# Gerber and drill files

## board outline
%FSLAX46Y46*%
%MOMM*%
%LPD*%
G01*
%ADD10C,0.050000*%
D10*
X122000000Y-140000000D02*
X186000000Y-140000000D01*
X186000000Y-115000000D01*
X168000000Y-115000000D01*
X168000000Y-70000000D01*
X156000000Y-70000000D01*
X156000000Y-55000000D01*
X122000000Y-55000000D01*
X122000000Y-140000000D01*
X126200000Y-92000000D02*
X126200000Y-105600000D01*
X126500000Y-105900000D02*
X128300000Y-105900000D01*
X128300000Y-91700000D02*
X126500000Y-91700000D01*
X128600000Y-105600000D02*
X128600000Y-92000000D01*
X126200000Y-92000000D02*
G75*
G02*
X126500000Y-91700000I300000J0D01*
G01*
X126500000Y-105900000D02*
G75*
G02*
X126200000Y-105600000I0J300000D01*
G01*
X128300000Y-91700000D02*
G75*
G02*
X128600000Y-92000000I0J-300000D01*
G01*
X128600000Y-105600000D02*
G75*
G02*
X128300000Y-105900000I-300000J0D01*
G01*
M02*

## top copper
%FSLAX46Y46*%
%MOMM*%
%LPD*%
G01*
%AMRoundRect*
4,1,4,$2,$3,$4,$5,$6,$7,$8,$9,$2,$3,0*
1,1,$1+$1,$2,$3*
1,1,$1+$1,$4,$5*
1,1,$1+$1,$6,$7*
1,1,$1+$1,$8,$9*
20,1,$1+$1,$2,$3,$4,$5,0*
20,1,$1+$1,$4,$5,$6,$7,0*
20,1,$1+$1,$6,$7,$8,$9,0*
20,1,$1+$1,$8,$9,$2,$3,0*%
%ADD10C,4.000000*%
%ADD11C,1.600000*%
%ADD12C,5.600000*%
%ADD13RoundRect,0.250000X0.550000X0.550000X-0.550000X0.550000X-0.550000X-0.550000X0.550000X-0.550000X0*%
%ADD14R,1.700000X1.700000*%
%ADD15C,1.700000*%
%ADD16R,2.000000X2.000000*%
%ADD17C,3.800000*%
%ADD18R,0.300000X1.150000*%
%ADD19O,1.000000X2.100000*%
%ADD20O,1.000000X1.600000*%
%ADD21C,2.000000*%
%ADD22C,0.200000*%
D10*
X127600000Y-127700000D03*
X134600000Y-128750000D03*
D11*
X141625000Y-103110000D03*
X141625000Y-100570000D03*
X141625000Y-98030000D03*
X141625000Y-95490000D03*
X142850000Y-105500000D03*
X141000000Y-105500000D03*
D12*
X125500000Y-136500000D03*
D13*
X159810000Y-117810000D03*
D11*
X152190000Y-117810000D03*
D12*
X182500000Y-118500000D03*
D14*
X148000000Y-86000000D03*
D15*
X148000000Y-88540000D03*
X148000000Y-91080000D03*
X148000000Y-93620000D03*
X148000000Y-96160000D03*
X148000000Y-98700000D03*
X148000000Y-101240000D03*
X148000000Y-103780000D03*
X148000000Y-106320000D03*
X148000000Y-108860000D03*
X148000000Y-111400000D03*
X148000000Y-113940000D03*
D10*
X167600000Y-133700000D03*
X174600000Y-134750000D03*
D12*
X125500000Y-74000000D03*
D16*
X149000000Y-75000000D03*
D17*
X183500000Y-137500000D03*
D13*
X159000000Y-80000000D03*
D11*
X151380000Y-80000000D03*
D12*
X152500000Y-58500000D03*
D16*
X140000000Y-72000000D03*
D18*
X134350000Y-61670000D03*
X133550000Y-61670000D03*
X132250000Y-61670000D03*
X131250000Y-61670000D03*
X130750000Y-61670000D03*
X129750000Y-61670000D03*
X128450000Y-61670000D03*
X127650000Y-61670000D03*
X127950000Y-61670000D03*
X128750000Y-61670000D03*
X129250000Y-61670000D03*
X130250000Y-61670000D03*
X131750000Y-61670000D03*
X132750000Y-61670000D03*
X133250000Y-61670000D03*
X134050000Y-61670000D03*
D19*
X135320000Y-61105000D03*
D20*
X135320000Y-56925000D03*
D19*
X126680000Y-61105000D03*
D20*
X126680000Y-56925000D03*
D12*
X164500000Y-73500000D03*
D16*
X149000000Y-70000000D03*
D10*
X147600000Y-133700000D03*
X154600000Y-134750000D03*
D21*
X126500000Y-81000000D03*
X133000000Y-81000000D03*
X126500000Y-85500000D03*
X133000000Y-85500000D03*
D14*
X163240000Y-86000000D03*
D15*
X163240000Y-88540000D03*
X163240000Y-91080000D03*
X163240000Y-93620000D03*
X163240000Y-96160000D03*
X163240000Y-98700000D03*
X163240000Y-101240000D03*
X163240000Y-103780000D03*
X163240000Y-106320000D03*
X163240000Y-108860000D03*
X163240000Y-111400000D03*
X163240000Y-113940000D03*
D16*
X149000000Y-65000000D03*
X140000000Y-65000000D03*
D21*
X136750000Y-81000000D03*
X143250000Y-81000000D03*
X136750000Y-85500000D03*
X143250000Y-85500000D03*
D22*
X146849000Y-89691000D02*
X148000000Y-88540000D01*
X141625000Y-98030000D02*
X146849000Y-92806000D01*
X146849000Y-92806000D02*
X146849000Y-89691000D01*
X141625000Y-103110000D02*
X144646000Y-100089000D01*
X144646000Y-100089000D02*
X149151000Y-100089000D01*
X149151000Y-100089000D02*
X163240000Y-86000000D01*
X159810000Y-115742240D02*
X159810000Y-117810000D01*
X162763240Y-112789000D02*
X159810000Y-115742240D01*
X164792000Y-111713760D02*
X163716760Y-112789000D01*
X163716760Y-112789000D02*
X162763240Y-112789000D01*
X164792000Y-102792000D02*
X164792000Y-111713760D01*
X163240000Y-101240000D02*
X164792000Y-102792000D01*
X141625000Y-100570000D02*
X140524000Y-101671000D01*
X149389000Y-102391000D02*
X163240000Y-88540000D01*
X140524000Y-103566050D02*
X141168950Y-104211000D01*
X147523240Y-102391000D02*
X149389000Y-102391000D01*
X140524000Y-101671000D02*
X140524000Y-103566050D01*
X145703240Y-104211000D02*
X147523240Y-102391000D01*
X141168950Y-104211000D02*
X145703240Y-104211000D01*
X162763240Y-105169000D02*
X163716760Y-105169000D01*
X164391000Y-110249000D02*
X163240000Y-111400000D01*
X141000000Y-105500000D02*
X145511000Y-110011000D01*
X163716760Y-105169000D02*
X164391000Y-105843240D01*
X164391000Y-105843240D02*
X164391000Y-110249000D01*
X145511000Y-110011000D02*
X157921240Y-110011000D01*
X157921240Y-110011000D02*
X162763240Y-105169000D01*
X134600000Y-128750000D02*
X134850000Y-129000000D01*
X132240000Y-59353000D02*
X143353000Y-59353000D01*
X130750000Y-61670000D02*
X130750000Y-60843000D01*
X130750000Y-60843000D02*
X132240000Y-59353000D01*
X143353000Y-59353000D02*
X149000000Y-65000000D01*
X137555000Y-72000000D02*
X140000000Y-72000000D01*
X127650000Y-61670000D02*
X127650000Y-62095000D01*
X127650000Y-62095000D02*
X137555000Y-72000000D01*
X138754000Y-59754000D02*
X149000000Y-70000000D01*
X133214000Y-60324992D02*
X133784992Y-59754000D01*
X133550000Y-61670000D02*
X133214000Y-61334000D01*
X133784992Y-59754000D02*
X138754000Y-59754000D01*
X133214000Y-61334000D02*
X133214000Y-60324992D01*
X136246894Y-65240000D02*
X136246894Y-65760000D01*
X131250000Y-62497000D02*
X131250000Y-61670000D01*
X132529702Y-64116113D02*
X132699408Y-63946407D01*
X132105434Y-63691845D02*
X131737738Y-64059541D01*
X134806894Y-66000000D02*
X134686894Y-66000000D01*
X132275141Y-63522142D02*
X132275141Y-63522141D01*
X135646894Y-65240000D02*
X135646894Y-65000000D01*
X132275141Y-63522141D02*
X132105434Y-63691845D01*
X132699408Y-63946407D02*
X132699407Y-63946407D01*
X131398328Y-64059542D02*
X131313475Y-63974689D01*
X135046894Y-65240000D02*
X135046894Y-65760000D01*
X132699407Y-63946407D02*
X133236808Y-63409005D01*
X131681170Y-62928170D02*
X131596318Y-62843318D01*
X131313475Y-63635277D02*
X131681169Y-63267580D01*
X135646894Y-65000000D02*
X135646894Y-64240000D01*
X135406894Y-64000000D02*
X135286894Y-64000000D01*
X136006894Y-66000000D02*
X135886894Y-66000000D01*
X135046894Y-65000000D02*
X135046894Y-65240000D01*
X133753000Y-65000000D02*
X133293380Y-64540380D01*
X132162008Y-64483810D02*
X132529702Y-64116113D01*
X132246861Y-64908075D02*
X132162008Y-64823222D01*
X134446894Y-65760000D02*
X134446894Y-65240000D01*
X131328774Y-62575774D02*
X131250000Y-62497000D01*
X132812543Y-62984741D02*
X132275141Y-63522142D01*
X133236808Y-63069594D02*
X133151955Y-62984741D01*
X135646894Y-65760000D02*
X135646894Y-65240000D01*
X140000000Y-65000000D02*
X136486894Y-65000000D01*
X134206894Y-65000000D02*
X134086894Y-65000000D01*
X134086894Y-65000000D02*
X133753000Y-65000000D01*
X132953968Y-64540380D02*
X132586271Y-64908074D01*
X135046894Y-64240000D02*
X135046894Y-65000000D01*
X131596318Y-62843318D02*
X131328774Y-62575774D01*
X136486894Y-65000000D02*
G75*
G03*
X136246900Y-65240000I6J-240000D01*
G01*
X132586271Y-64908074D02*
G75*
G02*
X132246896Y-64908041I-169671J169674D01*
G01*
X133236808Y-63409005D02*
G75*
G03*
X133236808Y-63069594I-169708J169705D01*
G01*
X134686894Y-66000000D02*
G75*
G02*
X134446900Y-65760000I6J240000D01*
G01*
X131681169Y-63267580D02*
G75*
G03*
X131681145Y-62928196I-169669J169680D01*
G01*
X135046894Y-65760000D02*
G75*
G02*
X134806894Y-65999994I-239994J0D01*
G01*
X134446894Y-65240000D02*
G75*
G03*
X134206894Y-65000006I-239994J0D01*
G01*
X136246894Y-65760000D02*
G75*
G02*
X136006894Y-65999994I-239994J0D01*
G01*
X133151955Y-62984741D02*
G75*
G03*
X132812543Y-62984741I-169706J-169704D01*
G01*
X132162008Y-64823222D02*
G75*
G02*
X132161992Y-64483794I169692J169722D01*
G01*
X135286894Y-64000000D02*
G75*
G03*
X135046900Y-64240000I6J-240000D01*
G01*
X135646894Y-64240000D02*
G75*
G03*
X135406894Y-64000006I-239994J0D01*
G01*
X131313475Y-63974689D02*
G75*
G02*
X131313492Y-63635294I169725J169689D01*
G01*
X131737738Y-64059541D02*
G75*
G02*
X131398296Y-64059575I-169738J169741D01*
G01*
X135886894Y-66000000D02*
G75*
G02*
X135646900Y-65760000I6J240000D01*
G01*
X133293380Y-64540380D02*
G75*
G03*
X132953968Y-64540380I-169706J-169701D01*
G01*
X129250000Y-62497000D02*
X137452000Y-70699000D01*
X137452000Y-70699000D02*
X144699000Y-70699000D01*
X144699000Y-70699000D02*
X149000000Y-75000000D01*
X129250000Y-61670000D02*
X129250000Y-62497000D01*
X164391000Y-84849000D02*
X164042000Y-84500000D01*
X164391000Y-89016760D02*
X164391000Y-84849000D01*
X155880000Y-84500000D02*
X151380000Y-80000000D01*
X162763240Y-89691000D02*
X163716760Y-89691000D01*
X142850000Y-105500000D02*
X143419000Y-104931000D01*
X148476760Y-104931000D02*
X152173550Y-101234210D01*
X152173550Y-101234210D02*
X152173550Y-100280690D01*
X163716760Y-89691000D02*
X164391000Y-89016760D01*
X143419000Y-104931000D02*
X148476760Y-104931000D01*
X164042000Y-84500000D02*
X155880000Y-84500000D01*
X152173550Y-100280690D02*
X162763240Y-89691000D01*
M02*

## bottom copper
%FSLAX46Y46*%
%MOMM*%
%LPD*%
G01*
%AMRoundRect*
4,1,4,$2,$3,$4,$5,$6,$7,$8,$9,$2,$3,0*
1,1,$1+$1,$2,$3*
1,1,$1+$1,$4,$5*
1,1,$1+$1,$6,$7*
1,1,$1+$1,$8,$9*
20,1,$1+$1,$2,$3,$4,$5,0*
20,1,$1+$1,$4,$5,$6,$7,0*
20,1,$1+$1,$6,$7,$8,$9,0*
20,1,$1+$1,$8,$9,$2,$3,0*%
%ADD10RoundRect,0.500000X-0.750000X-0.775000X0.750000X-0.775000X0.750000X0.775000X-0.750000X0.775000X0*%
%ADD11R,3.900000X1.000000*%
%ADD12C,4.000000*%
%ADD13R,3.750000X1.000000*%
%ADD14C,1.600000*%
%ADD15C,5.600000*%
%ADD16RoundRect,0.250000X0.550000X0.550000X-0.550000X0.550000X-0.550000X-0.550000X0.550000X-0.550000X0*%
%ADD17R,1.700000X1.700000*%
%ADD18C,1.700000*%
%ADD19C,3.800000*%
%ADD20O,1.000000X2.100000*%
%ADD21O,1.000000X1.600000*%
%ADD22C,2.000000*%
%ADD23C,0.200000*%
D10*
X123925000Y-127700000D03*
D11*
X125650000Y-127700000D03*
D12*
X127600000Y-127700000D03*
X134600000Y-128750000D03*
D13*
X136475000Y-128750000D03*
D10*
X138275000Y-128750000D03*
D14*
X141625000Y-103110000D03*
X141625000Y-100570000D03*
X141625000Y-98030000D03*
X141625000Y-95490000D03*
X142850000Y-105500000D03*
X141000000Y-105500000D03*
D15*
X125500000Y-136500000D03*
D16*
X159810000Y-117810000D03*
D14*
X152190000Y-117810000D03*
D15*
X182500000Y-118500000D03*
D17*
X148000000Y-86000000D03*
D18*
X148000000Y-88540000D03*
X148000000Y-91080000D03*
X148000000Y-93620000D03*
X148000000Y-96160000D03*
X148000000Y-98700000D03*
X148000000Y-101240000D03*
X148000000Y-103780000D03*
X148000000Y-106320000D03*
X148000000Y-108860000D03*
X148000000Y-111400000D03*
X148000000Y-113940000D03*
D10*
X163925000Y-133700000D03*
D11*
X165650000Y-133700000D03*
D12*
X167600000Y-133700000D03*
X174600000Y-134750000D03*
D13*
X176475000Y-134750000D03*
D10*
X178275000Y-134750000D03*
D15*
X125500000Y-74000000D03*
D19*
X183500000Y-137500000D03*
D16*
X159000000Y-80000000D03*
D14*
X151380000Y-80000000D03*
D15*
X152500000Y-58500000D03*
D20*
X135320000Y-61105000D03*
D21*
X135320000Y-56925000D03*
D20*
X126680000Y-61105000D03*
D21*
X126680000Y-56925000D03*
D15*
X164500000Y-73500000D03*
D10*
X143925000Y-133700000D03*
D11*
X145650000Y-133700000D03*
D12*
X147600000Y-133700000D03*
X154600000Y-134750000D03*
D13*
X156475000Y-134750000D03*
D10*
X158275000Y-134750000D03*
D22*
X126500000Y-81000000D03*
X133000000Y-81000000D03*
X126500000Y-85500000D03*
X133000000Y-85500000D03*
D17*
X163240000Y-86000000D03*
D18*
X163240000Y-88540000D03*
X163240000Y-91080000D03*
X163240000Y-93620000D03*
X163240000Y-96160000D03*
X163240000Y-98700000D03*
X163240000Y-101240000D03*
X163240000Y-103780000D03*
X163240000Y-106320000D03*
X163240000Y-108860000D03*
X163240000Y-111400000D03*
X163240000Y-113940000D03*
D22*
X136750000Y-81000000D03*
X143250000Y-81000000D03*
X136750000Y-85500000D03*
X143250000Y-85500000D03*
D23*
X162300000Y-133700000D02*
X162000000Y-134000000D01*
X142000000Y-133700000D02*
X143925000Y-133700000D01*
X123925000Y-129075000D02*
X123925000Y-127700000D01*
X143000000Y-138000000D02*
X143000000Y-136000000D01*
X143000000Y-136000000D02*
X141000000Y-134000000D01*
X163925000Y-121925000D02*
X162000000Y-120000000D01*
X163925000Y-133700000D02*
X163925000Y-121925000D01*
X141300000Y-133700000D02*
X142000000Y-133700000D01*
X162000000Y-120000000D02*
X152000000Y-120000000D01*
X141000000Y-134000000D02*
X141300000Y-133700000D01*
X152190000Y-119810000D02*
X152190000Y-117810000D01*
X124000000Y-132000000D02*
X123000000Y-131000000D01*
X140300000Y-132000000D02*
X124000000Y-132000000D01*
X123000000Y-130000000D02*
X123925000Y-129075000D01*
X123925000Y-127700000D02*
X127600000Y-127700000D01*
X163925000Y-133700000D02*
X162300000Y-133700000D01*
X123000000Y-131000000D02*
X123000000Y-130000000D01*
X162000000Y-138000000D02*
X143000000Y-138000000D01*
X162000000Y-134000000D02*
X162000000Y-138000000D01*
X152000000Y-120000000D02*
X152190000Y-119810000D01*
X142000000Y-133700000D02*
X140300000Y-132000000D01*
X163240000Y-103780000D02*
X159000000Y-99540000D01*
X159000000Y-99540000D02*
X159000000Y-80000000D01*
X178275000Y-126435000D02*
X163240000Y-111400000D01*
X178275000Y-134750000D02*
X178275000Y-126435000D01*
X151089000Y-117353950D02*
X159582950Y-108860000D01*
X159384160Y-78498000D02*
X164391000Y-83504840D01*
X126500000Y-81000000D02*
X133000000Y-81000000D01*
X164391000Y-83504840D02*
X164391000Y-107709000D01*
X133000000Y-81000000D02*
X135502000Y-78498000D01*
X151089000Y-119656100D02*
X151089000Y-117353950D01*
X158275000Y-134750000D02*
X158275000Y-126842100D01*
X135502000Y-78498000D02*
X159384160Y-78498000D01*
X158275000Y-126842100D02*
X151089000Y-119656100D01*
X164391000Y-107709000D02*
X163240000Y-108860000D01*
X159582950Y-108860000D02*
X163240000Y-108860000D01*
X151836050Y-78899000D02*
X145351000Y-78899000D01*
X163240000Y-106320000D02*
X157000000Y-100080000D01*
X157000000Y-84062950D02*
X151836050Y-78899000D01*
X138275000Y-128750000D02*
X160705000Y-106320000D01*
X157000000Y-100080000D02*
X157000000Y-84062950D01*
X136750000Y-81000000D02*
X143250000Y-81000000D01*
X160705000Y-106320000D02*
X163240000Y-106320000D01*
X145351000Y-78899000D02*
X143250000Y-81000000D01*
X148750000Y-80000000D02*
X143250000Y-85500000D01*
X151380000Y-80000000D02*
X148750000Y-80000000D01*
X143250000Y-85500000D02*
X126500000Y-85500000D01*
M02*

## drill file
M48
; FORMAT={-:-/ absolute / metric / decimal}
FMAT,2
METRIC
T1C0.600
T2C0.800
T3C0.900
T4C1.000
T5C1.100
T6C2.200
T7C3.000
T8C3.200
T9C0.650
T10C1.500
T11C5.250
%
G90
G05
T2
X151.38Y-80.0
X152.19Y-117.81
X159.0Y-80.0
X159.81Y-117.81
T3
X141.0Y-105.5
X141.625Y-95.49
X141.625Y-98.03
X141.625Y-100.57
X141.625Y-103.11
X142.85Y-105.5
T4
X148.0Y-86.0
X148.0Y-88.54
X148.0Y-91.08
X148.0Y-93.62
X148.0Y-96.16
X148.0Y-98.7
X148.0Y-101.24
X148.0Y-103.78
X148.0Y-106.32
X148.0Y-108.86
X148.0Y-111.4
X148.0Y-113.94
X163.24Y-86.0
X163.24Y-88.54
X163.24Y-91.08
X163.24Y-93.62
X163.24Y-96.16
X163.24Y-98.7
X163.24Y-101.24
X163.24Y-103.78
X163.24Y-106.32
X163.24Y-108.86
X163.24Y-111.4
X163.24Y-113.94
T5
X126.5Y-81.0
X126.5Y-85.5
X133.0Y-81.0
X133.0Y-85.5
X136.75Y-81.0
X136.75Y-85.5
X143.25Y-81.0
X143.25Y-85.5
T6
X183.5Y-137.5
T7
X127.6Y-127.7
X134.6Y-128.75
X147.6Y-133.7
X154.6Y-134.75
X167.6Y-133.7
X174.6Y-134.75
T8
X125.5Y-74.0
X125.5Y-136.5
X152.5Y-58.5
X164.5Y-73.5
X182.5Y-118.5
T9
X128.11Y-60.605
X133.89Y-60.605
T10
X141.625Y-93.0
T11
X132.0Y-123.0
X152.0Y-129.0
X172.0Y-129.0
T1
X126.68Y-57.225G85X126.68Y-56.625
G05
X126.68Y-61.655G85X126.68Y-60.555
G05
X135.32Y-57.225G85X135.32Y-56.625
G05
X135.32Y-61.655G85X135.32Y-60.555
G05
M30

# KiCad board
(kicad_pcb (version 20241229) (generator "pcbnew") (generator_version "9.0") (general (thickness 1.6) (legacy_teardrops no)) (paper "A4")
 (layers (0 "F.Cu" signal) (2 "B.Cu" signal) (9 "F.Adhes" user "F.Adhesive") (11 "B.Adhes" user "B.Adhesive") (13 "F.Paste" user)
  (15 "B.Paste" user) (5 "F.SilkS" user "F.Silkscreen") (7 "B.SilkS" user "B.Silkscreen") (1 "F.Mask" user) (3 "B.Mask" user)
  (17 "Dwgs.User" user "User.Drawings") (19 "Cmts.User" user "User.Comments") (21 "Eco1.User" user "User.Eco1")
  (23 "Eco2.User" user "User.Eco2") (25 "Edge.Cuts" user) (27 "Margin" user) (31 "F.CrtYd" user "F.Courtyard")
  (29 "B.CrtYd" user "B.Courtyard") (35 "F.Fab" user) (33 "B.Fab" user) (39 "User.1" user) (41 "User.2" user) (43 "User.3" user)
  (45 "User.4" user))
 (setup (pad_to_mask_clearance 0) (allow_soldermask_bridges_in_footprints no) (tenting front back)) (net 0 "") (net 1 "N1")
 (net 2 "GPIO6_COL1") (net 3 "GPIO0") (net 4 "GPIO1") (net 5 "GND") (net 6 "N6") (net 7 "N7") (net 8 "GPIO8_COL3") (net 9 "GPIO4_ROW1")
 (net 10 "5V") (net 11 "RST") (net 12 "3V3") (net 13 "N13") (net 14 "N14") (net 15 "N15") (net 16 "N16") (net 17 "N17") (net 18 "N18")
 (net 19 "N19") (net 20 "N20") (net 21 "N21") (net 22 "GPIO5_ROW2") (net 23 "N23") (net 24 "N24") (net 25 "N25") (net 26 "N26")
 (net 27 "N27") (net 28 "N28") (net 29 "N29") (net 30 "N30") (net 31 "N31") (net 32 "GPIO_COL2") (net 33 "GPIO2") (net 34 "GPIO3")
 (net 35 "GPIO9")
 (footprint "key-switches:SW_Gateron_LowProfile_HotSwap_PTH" (layer "F.Cu") (at 132 123)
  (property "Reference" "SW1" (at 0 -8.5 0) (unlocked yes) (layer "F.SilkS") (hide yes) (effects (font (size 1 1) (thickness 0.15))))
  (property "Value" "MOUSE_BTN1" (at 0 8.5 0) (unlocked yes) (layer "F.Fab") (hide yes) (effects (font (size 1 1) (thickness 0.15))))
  (pad "" np_thru_hole circle (at 0 0) (size 5.25 5.25) (drill 5.25) (layers "*.Mask"))
  (pad "1" smd roundrect (at -8.075 4.7) (size 2.5 2.55) (layers "B.Cu" "B.Mask" "B.Paste") (roundrect_rratio 0.2) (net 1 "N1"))
  (pad "1" smd rect (at -6.35 4.7) (size 3.9 1) (layers "B.Cu") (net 1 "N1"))
  (pad "1" thru_hole circle (at -4.4 4.7) (size 4 4) (drill 3) (layers "*.Cu" "B.Mask") (remove_unused_layers no) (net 1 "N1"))
  (pad "2" thru_hole circle (at 2.6 5.75) (size 4 4) (drill 3) (layers "*.Cu" "B.Mask") (remove_unused_layers no) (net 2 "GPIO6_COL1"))
  (pad "2" smd rect (at 4.475 5.75) (size 3.75 1) (layers "B.Cu") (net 2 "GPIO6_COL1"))
  (pad "2" smd roundrect (at 6.275 5.75) (size 2.5 2.55) (layers "B.Cu" "B.Mask" "B.Paste") (roundrect_rratio 0.2) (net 2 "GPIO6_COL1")))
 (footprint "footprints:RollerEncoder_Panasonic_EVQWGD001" (layer "F.Cu") (at 136 99.3 180)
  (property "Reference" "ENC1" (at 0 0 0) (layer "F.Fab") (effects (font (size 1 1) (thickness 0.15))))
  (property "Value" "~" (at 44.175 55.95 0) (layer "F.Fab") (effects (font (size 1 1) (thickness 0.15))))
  (fp_line (start 9.8 7.3) (end 9.8 -6.3) (stroke (width 0.05) (type solid)) (layer "Edge.Cuts"))
  (fp_line (start 9.5 -6.6) (end 7.7 -6.6) (stroke (width 0.05) (type solid)) (layer "Edge.Cuts"))
  (fp_line (start 7.7 7.6) (end 9.5 7.6) (stroke (width 0.05) (type solid)) (layer "Edge.Cuts"))
  (fp_line (start 7.4 -6.3) (end 7.4 7.3) (stroke (width 0.05) (type solid)) (layer "Edge.Cuts"))
  (fp_arc (start 9.8 7.3) (mid 9.712132 7.512132) (end 9.5 7.6) (stroke (width 0.05) (type solid)) (layer "Edge.Cuts"))
  (fp_arc (start 9.5 -6.6) (mid 9.712132 -6.512132) (end 9.8 -6.3) (stroke (width 0.05) (type solid)) (layer "Edge.Cuts"))
  (fp_arc (start 7.7 7.6) (mid 7.487868 7.512132) (end 7.4 7.3) (stroke (width 0.05) (type solid)) (layer "Edge.Cuts"))
  (fp_arc (start 7.4 -6.3) (mid 7.487868 -6.512132) (end 7.7 -6.6) (stroke (width 0.05) (type solid)) (layer "Edge.Cuts"))
  (pad "" np_thru_hole circle (at -5.625 6.3 180) (size 1.5 1.5) (drill 1.5) (layers "*.Cu" "*.Mask"))
  (pad "A" thru_hole circle (at -5.625 -3.81 180) (size 1.6 1.6) (drill 0.9) (layers "*.Cu" "*.Mask") (remove_unused_layers no)
   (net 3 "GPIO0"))
  (pad "B" thru_hole circle (at -5.625 -1.27 180) (size 1.6 1.6) (drill 0.9) (layers "*.Cu" "*.Mask") (remove_unused_layers no)
   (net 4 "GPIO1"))
  (pad "C" thru_hole circle (at -5.625 1.27 180) (size 1.6 1.6) (drill 0.9) (layers "*.Cu" "*.Mask") (remove_unused_layers no) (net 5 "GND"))
  (pad "D" thru_hole circle (at -5.625 3.81 180) (size 1.6 1.6) (drill 0.9) (layers "*.Cu" "*.Mask") (remove_unused_layers no) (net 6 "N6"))
  (pad "S1" thru_hole circle (at -6.85 -6.2 180) (size 1.6 1.6) (drill 0.9) (layers "*.Cu" "*.Mask") (remove_unused_layers no) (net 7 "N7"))
  (pad "S2" thru_hole circle (at -5 -6.2 180) (size 1.6 1.6) (drill 0.9) (layers "*.Cu" "*.Mask") (remove_unused_layers no)
   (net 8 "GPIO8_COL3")))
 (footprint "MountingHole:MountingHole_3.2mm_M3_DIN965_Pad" (layer "F.Cu") (at 125.5 136.5)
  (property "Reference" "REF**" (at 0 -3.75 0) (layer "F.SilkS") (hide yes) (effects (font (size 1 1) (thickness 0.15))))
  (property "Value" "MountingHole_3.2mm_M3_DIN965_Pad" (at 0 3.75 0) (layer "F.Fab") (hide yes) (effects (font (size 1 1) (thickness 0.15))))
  (pad "1" thru_hole circle (at 0 0) (size 5.6 5.6) (drill 3.2) (layers "*.Cu" "*.Mask") (remove_unused_layers no) (zone_connect 2)))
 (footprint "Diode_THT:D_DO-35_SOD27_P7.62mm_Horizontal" (layer "F.Cu") (at 159.81 117.81 180)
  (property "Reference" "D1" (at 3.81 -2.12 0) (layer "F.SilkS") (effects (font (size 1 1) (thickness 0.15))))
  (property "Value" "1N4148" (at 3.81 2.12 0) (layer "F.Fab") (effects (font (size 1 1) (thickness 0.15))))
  (pad "1" thru_hole roundrect (at 0 0 180) (size 1.6 1.6) (drill 0.8) (layers "*.Cu" "*.Mask") (remove_unused_layers no)
   (roundrect_rratio 0.15625) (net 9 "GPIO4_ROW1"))
  (pad "2" thru_hole circle (at 7.62 0 180) (size 1.6 1.6) (drill 0.8) (layers "*.Cu" "*.Mask") (remove_unused_layers no) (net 1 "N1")))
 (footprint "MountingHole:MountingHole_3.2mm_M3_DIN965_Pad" (layer "F.Cu") (at 182.5 118.5)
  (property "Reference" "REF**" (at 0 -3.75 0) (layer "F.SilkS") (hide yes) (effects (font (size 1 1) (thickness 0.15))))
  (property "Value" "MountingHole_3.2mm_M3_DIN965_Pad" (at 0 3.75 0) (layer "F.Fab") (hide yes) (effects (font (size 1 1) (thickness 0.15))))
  (pad "1" thru_hole circle (at 0 0) (size 5.6 5.6) (drill 3.2) (layers "*.Cu" "*.Mask") (remove_unused_layers no) (zone_connect 2)))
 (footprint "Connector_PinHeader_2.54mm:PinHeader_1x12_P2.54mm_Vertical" (layer "F.Cu") (at 148 86)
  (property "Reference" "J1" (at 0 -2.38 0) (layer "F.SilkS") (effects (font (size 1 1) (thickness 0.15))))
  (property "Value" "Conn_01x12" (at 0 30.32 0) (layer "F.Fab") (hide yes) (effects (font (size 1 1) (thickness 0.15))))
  (pad "1" thru_hole rect (at 0 0) (size 1.7 1.7) (drill 1) (layers "*.Cu" "*.Mask") (remove_unused_layers no) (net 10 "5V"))
  (pad "2" thru_hole circle (at 0 2.54) (size 1.7 1.7) (drill 1) (layers "*.Cu" "*.Mask") (remove_unused_layers no) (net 5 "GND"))
  (pad "3" thru_hole circle (at 0 5.08) (size 1.7 1.7) (drill 1) (layers "*.Cu" "*.Mask") (remove_unused_layers no) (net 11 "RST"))
  (pad "4" thru_hole circle (at 0 7.62) (size 1.7 1.7) (drill 1) (layers "*.Cu" "*.Mask") (remove_unused_layers no) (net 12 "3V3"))
  (pad "5" thru_hole circle (at 0 10.16) (size 1.7 1.7) (drill 1) (layers "*.Cu" "*.Mask") (remove_unused_layers no) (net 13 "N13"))
  (pad "6" thru_hole circle (at 0 12.7) (size 1.7 1.7) (drill 1) (layers "*.Cu" "*.Mask") (remove_unused_layers no) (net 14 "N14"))
  (pad "7" thru_hole circle (at 0 15.24) (size 1.7 1.7) (drill 1) (layers "*.Cu" "*.Mask") (remove_unused_layers no) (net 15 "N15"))
  (pad "8" thru_hole circle (at 0 17.78) (size 1.7 1.7) (drill 1) (layers "*.Cu" "*.Mask") (remove_unused_layers no) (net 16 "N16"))
  (pad "9" thru_hole circle (at 0 20.32) (size 1.7 1.7) (drill 1) (layers "*.Cu" "*.Mask") (remove_unused_layers no) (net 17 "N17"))
  (pad "10" thru_hole circle (at 0 22.86) (size 1.7 1.7) (drill 1) (layers "*.Cu" "*.Mask") (remove_unused_layers no) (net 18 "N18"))
  (pad "11" thru_hole circle (at 0 25.4) (size 1.7 1.7) (drill 1) (layers "*.Cu" "*.Mask") (remove_unused_layers no) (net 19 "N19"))
  (pad "12" thru_hole circle (at 0 27.94) (size 1.7 1.7) (drill 1) (layers "*.Cu" "*.Mask") (remove_unused_layers no) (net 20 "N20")))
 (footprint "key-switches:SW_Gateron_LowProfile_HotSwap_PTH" (layer "F.Cu") (at 172 129)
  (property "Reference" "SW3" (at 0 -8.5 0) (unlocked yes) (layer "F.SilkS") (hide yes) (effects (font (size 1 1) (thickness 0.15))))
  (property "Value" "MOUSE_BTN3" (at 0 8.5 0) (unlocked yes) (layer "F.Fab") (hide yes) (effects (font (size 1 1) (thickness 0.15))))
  (pad "" np_thru_hole circle (at 0 0) (size 5.25 5.25) (drill 5.25) (layers "*.Mask"))
  (pad "1" smd roundrect (at -8.075 4.7) (size 2.5 2.55) (layers "B.Cu" "B.Mask" "B.Paste") (roundrect_rratio 0.2) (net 1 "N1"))
  (pad "1" smd rect (at -6.35 4.7) (size 3.9 1) (layers "B.Cu") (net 1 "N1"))
  (pad "1" thru_hole circle (at -4.4 4.7) (size 4 4) (drill 3) (layers "*.Cu" "B.Mask") (remove_unused_layers no) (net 1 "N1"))
  (pad "2" thru_hole circle (at 2.6 5.75) (size 4 4) (drill 3) (layers "*.Cu" "B.Mask") (remove_unused_layers no) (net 8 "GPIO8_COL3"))
  (pad "2" smd rect (at 4.475 5.75) (size 3.75 1) (layers "B.Cu") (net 8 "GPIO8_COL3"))
  (pad "2" smd roundrect (at 6.275 5.75) (size 2.5 2.55) (layers "B.Cu" "B.Mask" "B.Paste") (roundrect_rratio 0.2) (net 8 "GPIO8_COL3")))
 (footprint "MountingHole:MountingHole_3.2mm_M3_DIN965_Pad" (layer "F.Cu") (at 125.5 74)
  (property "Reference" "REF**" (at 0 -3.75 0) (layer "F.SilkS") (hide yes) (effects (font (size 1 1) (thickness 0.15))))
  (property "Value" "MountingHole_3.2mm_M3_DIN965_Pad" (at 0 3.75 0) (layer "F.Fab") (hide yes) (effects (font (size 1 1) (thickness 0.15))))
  (pad "1" thru_hole circle (at 0 0) (size 5.6 5.6) (drill 3.2) (layers "*.Cu" "*.Mask") (remove_unused_layers no) (zone_connect 2)))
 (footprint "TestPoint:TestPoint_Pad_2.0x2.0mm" (layer "F.Cu") (at 149 75)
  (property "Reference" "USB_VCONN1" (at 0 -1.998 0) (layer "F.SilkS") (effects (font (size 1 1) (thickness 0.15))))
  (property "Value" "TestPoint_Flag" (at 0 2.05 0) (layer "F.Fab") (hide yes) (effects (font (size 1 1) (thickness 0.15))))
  (pad "1" smd rect (at 0 0) (size 2 2) (layers "F.Cu" "F.Mask") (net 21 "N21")))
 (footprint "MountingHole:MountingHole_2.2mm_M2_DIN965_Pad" (layer "F.Cu") (at 183.5 137.5)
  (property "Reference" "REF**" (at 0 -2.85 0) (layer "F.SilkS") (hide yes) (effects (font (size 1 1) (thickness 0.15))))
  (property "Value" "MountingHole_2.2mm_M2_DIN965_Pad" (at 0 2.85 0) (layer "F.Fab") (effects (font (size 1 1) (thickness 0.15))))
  (pad "1" thru_hole circle (at 0 0) (size 3.8 3.8) (drill 2.2) (layers "*.Cu" "*.Mask") (remove_unused_layers no) (zone_connect 2)))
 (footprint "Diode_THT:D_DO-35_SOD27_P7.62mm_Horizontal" (layer "F.Cu") (at 159 80 180)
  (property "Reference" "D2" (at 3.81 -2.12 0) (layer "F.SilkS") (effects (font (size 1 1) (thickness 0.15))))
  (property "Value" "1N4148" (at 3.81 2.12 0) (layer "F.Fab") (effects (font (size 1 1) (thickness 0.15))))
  (pad "1" thru_hole roundrect (at 0 0 180) (size 1.6 1.6) (drill 0.8) (layers "*.Cu" "*.Mask") (remove_unused_layers no)
   (roundrect_rratio 0.15625) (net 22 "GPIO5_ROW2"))
  (pad "2" thru_hole circle (at 7.62 0 180) (size 1.6 1.6) (drill 0.8) (layers "*.Cu" "*.Mask") (remove_unused_layers no) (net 7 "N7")))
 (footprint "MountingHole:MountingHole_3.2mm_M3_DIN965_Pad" (layer "F.Cu") (at 152.5 58.5)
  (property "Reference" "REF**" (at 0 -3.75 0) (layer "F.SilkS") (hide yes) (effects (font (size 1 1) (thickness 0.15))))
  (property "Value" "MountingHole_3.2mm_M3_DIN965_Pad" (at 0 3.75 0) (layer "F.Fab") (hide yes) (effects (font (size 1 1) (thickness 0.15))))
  (pad "1" thru_hole circle (at 0 0) (size 5.6 5.6) (drill 3.2) (layers "*.Cu" "*.Mask") (remove_unused_layers no) (zone_connect 2)))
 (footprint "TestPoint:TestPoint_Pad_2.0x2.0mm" (layer "F.Cu") (at 140 72)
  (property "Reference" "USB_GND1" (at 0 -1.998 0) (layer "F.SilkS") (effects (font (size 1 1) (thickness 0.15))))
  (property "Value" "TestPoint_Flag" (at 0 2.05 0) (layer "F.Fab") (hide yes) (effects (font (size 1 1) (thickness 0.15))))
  (pad "1" smd rect (at 0 0) (size 2 2) (layers "F.Cu" "F.Mask") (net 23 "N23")))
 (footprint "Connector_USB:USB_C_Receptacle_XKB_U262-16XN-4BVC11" (layer "F.Cu") (at 131 58 180)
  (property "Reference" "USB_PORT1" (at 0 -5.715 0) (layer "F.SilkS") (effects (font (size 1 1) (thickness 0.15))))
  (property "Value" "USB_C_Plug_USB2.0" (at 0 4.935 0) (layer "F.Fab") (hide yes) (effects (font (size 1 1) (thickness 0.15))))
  (pad "" np_thru_hole circle (at -2.89 -2.605 180) (size 0.65 0.65) (drill 0.65) (layers "*.Cu" "*.Mask"))
  (pad "" np_thru_hole circle (at 2.89 -2.605 180) (size 0.65 0.65) (drill 0.65) (layers "*.Cu" "*.Mask"))
  (pad "A1" smd rect (at -3.35 -3.67 180) (size 0.3 1.15) (layers "F.Cu" "F.Mask" "F.Paste") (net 23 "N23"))
  (pad "A4" smd rect (at -2.55 -3.67 180) (size 0.3 1.15) (layers "F.Cu" "F.Mask" "F.Paste") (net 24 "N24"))
  (pad "A5" smd rect (at -1.25 -3.67 180) (size 0.3 1.15) (layers "F.Cu" "F.Mask" "F.Paste") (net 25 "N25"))
  (pad "A6" smd rect (at -0.25 -3.67 180) (size 0.3 1.15) (layers "F.Cu" "F.Mask" "F.Paste") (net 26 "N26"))
  (pad "A7" smd rect (at 0.25 -3.67 180) (size 0.3 1.15) (layers "F.Cu" "F.Mask" "F.Paste") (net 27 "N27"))
  (pad "A8" smd rect (at 1.25 -3.67 180) (size 0.3 1.15) (layers "F.Cu" "F.Mask" "F.Paste"))
  (pad "A9" smd rect (at 2.55 -3.67 180) (size 0.3 1.15) (layers "F.Cu" "F.Mask" "F.Paste") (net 24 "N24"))
  (pad "A12" smd rect (at 3.35 -3.67 180) (size 0.3 1.15) (layers "F.Cu" "F.Mask" "F.Paste") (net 23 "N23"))
  (pad "B1" smd rect (at 3.05 -3.67 180) (size 0.3 1.15) (layers "F.Cu" "F.Mask" "F.Paste") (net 23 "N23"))
  (pad "B4" smd rect (at 2.25 -3.67 180) (size 0.3 1.15) (layers "F.Cu" "F.Mask" "F.Paste") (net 24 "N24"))
  (pad "B5" smd rect (at 1.75 -3.67 180) (size 0.3 1.15) (layers "F.Cu" "F.Mask" "F.Paste") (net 21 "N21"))
  (pad "B6" smd rect (at 0.75 -3.67 180) (size 0.3 1.15) (layers "F.Cu" "F.Mask" "F.Paste"))
  (pad "B7" smd rect (at -0.75 -3.67 180) (size 0.3 1.15) (layers "F.Cu" "F.Mask" "F.Paste"))
  (pad "B8" smd rect (at -1.75 -3.67 180) (size 0.3 1.15) (layers "F.Cu" "F.Mask" "F.Paste"))
  (pad "B9" smd rect (at -2.25 -3.67 180) (size 0.3 1.15) (layers "F.Cu" "F.Mask" "F.Paste") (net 24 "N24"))
  (pad "B12" smd rect (at -3.05 -3.67 180) (size 0.3 1.15) (layers "F.Cu" "F.Mask" "F.Paste") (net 23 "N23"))
  (pad "S1" thru_hole oval (at -4.32 -3.105 180) (size 1 2.1) (drill oval 0.6 1.7) (layers "*.Cu" "*.Mask") (remove_unused_layers no)
   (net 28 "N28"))
  (pad "S1" thru_hole oval (at -4.32 1.075 180) (size 1 1.6) (drill oval 0.6 1.2) (layers "*.Cu" "*.Mask") (remove_unused_layers no)
   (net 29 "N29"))
  (pad "S1" thru_hole oval (at 4.32 -3.105 180) (size 1 2.1) (drill oval 0.6 1.7) (layers "*.Cu" "*.Mask") (remove_unused_layers no)
   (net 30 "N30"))
  (pad "S1" thru_hole oval (at 4.32 1.075 180) (size 1 1.6) (drill oval 0.6 1.2) (layers "*.Cu" "*.Mask") (remove_unused_layers no)
   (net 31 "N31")))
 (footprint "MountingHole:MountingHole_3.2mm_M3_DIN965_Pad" (layer "F.Cu") (at 164.5 73.5)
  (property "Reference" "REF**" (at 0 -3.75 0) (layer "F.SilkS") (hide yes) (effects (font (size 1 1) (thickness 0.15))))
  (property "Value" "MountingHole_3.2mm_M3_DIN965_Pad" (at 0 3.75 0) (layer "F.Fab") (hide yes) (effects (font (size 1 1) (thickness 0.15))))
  (pad "1" thru_hole circle (at 0 0) (size 5.6 5.6) (drill 3.2) (layers "*.Cu" "*.Mask") (remove_unused_layers no) (zone_connect 2)))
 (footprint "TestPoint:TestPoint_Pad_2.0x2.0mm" (layer "F.Cu") (at 149 70)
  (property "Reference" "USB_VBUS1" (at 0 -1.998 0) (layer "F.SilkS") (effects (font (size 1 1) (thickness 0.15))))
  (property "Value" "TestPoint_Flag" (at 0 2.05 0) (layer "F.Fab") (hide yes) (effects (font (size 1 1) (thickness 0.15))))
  (pad "1" smd rect (at 0 0) (size 2 2) (layers "F.Cu" "F.Mask") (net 24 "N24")))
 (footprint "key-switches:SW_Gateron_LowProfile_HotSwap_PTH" (layer "F.Cu") (at 152 129)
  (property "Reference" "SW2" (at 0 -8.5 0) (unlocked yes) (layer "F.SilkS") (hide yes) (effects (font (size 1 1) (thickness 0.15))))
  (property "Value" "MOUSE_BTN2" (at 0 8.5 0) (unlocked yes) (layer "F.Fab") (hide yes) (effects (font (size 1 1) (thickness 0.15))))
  (pad "" np_thru_hole circle (at 0 0) (size 5.25 5.25) (drill 5.25) (layers "*.Mask"))
  (pad "1" smd roundrect (at -8.075 4.7) (size 2.5 2.55) (layers "B.Cu" "B.Mask" "B.Paste") (roundrect_rratio 0.2) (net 1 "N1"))
  (pad "1" smd rect (at -6.35 4.7) (size 3.9 1) (layers "B.Cu") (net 1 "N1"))
  (pad "1" thru_hole circle (at -4.4 4.7) (size 4 4) (drill 3) (layers "*.Cu" "B.Mask") (remove_unused_layers no) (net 1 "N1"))
  (pad "2" thru_hole circle (at 2.6 5.75) (size 4 4) (drill 3) (layers "*.Cu" "B.Mask") (remove_unused_layers no) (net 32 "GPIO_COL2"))
  (pad "2" smd rect (at 4.475 5.75) (size 3.75 1) (layers "B.Cu") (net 32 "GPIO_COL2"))
  (pad "2" smd roundrect (at 6.275 5.75) (size 2.5 2.55) (layers "B.Cu" "B.Mask" "B.Paste") (roundrect_rratio 0.2) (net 32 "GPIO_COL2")))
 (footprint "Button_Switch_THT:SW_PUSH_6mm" (layer "F.Cu") (at 126.5 81)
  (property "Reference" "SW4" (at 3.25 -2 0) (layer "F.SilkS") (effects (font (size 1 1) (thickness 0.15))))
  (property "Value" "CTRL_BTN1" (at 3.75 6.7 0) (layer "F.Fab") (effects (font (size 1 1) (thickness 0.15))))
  (pad "1" thru_hole circle (at 0 0 90) (size 2 2) (drill 1.1) (layers "*.Cu" "*.Mask") (remove_unused_layers no) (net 32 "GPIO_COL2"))
  (pad "1" thru_hole circle (at 6.5 0 90) (size 2 2) (drill 1.1) (layers "*.Cu" "*.Mask") (remove_unused_layers no) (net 32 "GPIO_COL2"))
  (pad "2" thru_hole circle (at 0 4.5 90) (size 2 2) (drill 1.1) (layers "*.Cu" "*.Mask") (remove_unused_layers no) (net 7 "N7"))
  (pad "2" thru_hole circle (at 6.5 4.5 90) (size 2 2) (drill 1.1) (layers "*.Cu" "*.Mask") (remove_unused_layers no) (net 7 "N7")))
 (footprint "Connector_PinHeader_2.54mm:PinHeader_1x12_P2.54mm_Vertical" (layer "F.Cu") (at 163.24 86)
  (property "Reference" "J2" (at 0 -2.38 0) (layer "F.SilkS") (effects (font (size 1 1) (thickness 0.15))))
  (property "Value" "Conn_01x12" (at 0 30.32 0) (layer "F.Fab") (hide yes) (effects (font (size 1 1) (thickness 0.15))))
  (pad "1" thru_hole rect (at 0 0) (size 1.7 1.7) (drill 1) (layers "*.Cu" "*.Mask") (remove_unused_layers no) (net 3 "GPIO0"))
  (pad "2" thru_hole circle (at 0 2.54) (size 1.7 1.7) (drill 1) (layers "*.Cu" "*.Mask") (remove_unused_layers no) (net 4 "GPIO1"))
  (pad "3" thru_hole circle (at 0 5.08) (size 1.7 1.7) (drill 1) (layers "*.Cu" "*.Mask") (remove_unused_layers no) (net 5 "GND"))
  (pad "4" thru_hole circle (at 0 7.62) (size 1.7 1.7) (drill 1) (layers "*.Cu" "*.Mask") (remove_unused_layers no) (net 5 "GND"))
  (pad "5" thru_hole circle (at 0 10.16) (size 1.7 1.7) (drill 1) (layers "*.Cu" "*.Mask") (remove_unused_layers no) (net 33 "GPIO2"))
  (pad "6" thru_hole circle (at 0 12.7) (size 1.7 1.7) (drill 1) (layers "*.Cu" "*.Mask") (remove_unused_layers no) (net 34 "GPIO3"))
  (pad "7" thru_hole circle (at 0 15.24) (size 1.7 1.7) (drill 1) (layers "*.Cu" "*.Mask") (remove_unused_layers no) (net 9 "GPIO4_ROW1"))
  (pad "8" thru_hole circle (at 0 17.78) (size 1.7 1.7) (drill 1) (layers "*.Cu" "*.Mask") (remove_unused_layers no) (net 22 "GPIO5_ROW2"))
  (pad "9" thru_hole circle (at 0 20.32) (size 1.7 1.7) (drill 1) (layers "*.Cu" "*.Mask") (remove_unused_layers no) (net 2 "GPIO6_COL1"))
  (pad "10" thru_hole circle (at 0 22.86) (size 1.7 1.7) (drill 1) (layers "*.Cu" "*.Mask") (remove_unused_layers no) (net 32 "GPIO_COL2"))
  (pad "11" thru_hole circle (at 0 25.4) (size 1.7 1.7) (drill 1) (layers "*.Cu" "*.Mask") (remove_unused_layers no) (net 8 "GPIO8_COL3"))
  (pad "12" thru_hole circle (at 0 27.94) (size 1.7 1.7) (drill 1) (layers "*.Cu" "*.Mask") (remove_unused_layers no) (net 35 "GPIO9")))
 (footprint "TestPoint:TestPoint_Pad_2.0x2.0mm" (layer "F.Cu") (at 149 65)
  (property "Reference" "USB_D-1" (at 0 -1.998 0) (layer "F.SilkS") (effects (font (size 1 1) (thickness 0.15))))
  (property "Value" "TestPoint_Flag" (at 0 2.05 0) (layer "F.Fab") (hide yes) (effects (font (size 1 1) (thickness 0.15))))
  (pad "1" smd rect (at 0 0) (size 2 2) (layers "F.Cu" "F.Mask") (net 27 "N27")))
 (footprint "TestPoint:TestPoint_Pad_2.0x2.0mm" (layer "F.Cu") (at 140 65)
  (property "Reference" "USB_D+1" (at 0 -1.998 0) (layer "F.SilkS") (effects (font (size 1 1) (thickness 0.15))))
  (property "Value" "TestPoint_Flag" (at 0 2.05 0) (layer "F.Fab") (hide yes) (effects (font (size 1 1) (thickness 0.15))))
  (pad "1" smd rect (at 0 0) (size 2 2) (layers "F.Cu" "F.Mask") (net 26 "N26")))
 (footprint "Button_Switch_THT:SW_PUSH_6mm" (layer "F.Cu") (at 136.75 81)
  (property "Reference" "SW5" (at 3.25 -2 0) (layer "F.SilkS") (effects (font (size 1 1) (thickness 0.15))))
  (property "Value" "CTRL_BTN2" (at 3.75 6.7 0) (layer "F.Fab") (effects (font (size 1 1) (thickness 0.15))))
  (pad "1" thru_hole circle (at 0 0 90) (size 2 2) (drill 1.1) (layers "*.Cu" "*.Mask") (remove_unused_layers no) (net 2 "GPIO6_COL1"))
  (pad "1" thru_hole circle (at 6.5 0 90) (size 2 2) (drill 1.1) (layers "*.Cu" "*.Mask") (remove_unused_layers no) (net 2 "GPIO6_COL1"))
  (pad "2" thru_hole circle (at 0 4.5 90) (size 2 2) (drill 1.1) (layers "*.Cu" "*.Mask") (remove_unused_layers no) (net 7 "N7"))
  (pad "2" thru_hole circle (at 6.5 4.5 90) (size 2 2) (drill 1.1) (layers "*.Cu" "*.Mask") (remove_unused_layers no) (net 7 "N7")))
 (gr_poly
  (pts (xy 122 140) (xy 186 140) (xy 186 115) (xy 168 115) (xy 168 70) (xy 156 70) (xy 156 55) (xy 122 55))
  (stroke (width 0.05) (type solid)) (fill no) (layer "Edge.Cuts"))
 (segment (start 162.3 133.7) (end 162 134) (width 0.2) (layer "B.Cu") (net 1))
 (segment (start 142 133.7) (end 143.925 133.7) (width 0.2) (layer "B.Cu") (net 1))
 (segment (start 123.925 129.075) (end 123.925 127.7) (width 0.2) (layer "B.Cu") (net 1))
 (segment (start 143 138) (end 143 136) (width 0.2) (layer "B.Cu") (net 1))
 (segment (start 143 136) (end 141 134) (width 0.2) (layer "B.Cu") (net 1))
 (segment (start 163.925 121.925) (end 162 120) (width 0.2) (layer "B.Cu") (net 1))
 (segment (start 163.925 133.7) (end 163.925 121.925) (width 0.2) (layer "B.Cu") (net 1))
 (segment (start 141.3 133.7) (end 142 133.7) (width 0.2) (layer "B.Cu") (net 1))
 (segment (start 162 120) (end 152 120) (width 0.2) (layer "B.Cu") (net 1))
 (segment (start 141 134) (end 141.3 133.7) (width 0.2) (layer "B.Cu") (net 1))
 (segment (start 152.19 119.81) (end 152.19 117.81) (width 0.2) (layer "B.Cu") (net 1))
 (segment (start 124 132) (end 123 131) (width 0.2) (layer "B.Cu") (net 1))
 (segment (start 140.3 132) (end 124 132) (width 0.2) (layer "B.Cu") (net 1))
 (segment (start 123 130) (end 123.925 129.075) (width 0.2) (layer "B.Cu") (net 1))
 (segment (start 123.925 127.7) (end 127.6 127.7) (width 0.2) (layer "B.Cu") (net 1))
 (segment (start 163.925 133.7) (end 162.3 133.7) (width 0.2) (layer "B.Cu") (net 1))
 (segment (start 123 131) (end 123 130) (width 0.2) (layer "B.Cu") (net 1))
 (segment (start 162 138) (end 143 138) (width 0.2) (layer "B.Cu") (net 1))
 (segment (start 162 134) (end 162 138) (width 0.2) (layer "B.Cu") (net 1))
 (segment (start 152 120) (end 152.19 119.81) (width 0.2) (layer "B.Cu") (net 1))
 (segment (start 142 133.7) (end 140.3 132) (width 0.2) (layer "B.Cu") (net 1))
 (segment (start 146.849 89.691) (end 148 88.54) (width 0.2) (layer "F.Cu") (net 5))
 (segment (start 141.625 98.03) (end 146.849 92.806) (width 0.2) (layer "F.Cu") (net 5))
 (segment (start 146.849 92.806) (end 146.849 89.691) (width 0.2) (layer "F.Cu") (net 5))
 (segment (start 163.24 103.78) (end 159 99.54) (width 0.2) (layer "B.Cu") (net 22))
 (segment (start 159 99.54) (end 159 80) (width 0.2) (layer "B.Cu") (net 22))
 (segment (start 141.625 103.11) (end 144.646 100.089) (width 0.2) (layer "F.Cu") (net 3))
 (segment (start 144.646 100.089) (end 149.151 100.089) (width 0.2) (layer "F.Cu") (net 3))
 (segment (start 149.151 100.089) (end 163.24 86) (width 0.2) (layer "F.Cu") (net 3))
 (segment (start 159.81 115.74224) (end 159.81 117.81) (width 0.2) (layer "F.Cu") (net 9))
 (segment (start 162.76324 112.789) (end 159.81 115.74224) (width 0.2) (layer "F.Cu") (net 9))
 (segment (start 164.792 111.71376) (end 163.71676 112.789) (width 0.2) (layer "F.Cu") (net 9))
 (segment (start 163.71676 112.789) (end 162.76324 112.789) (width 0.2) (layer "F.Cu") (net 9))
 (segment (start 164.792 102.792) (end 164.792 111.71376) (width 0.2) (layer "F.Cu") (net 9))
 (segment (start 163.24 101.24) (end 164.792 102.792) (width 0.2) (layer "F.Cu") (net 9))
 (segment (start 141.625 100.57) (end 140.524 101.671) (width 0.2) (layer "F.Cu") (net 4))
 (segment (start 149.389 102.391) (end 163.24 88.54) (width 0.2) (layer "F.Cu") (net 4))
 (segment (start 140.524 103.56605) (end 141.16895 104.211) (width 0.2) (layer "F.Cu") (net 4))
 (segment (start 147.52324 102.391) (end 149.389 102.391) (width 0.2) (layer "F.Cu") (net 4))
 (segment (start 140.524 101.671) (end 140.524 103.56605) (width 0.2) (layer "F.Cu") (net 4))
 (segment (start 145.70324 104.211) (end 147.52324 102.391) (width 0.2) (layer "F.Cu") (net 4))
 (segment (start 141.16895 104.211) (end 145.70324 104.211) (width 0.2) (layer "F.Cu") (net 4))
 (segment (start 162.76324 105.169) (end 163.71676 105.169) (width 0.2) (layer "F.Cu") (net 8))
 (segment (start 164.391 110.249) (end 163.24 111.4) (width 0.2) (layer "F.Cu") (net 8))
 (segment (start 141 105.5) (end 145.511 110.011) (width 0.2) (layer "F.Cu") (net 8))
 (segment (start 163.71676 105.169) (end 164.391 105.84324) (width 0.2) (layer "F.Cu") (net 8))
 (segment (start 164.391 105.84324) (end 164.391 110.249) (width 0.2) (layer "F.Cu") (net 8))
 (segment (start 145.511 110.011) (end 157.92124 110.011) (width 0.2) (layer "F.Cu") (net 8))
 (segment (start 157.92124 110.011) (end 162.76324 105.169) (width 0.2) (layer "F.Cu") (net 8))
 (segment (start 178.275 126.435) (end 163.24 111.4) (width 0.2) (layer "B.Cu") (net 8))
 (segment (start 178.275 134.75) (end 178.275 126.435) (width 0.2) (layer "B.Cu") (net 8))
 (segment (start 151.089 117.35395) (end 159.58295 108.86) (width 0.2) (layer "B.Cu") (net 32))
 (segment (start 159.38416 78.498) (end 164.391 83.50484) (width 0.2) (layer "B.Cu") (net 32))
 (segment (start 126.5 81) (end 133 81) (width 0.2) (layer "B.Cu") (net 32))
 (segment (start 164.391 83.50484) (end 164.391 107.709) (width 0.2) (layer "B.Cu") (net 32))
 (segment (start 133 81) (end 135.502 78.498) (width 0.2) (layer "B.Cu") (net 32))
 (segment (start 151.089 119.6561) (end 151.089 117.35395) (width 0.2) (layer "B.Cu") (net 32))
 (segment (start 158.275 134.75) (end 158.275 126.8421) (width 0.2) (layer "B.Cu") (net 32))
 (segment (start 135.502 78.498) (end 159.38416 78.498) (width 0.2) (layer "B.Cu") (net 32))
 (segment (start 158.275 126.8421) (end 151.089 119.6561) (width 0.2) (layer "B.Cu") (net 32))
 (segment (start 164.391 107.709) (end 163.24 108.86) (width 0.2) (layer "B.Cu") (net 32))
 (segment (start 159.58295 108.86) (end 163.24 108.86) (width 0.2) (layer "B.Cu") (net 32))
 (segment (start 134.6 128.75) (end 134.85 129) (width 0.2) (layer "F.Cu") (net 2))
 (segment (start 151.83605 78.899) (end 145.351 78.899) (width 0.2) (layer "B.Cu") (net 2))
 (segment (start 163.24 106.32) (end 157 100.08) (width 0.2) (layer "B.Cu") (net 2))
 (segment (start 157 84.06295) (end 151.83605 78.899) (width 0.2) (layer "B.Cu") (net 2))
 (segment (start 138.275 128.75) (end 160.705 106.32) (width 0.2) (layer "B.Cu") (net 2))
 (segment (start 157 100.08) (end 157 84.06295) (width 0.2) (layer "B.Cu") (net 2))
 (segment (start 136.75 81) (end 143.25 81) (width 0.2) (layer "B.Cu") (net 2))
 (segment (start 160.705 106.32) (end 163.24 106.32) (width 0.2) (layer "B.Cu") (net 2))
 (segment (start 145.351 78.899) (end 143.25 81) (width 0.2) (layer "B.Cu") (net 2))
 (segment (start 132.24 59.353) (end 143.353 59.353) (width 0.2) (layer "F.Cu") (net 27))
 (segment (start 130.75 61.67) (end 130.75 60.843) (width 0.2) (layer "F.Cu") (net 27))
 (segment (start 130.75 60.843) (end 132.24 59.353) (width 0.2) (layer "F.Cu") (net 27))
 (segment (start 143.353 59.353) (end 149 65) (width 0.2) (layer "F.Cu") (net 27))
 (segment (start 137.555 72) (end 140 72) (width 0.2) (layer "F.Cu") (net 23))
 (segment (start 127.65 61.67) (end 127.65 62.095) (width 0.2) (layer "F.Cu") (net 23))
 (segment (start 127.65 62.095) (end 137.555 72) (width 0.2) (layer "F.Cu") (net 23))
 (segment (start 138.754 59.754) (end 149 70) (width 0.2) (layer "F.Cu") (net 24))
 (segment (start 133.214 60.324992) (end 133.784992 59.754) (width 0.2) (layer "F.Cu") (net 24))
 (segment (start 133.55 61.67) (end 133.214 61.334) (width 0.2) (layer "F.Cu") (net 24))
 (segment (start 133.784992 59.754) (end 138.754 59.754) (width 0.2) (layer "F.Cu") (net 24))
 (segment (start 133.214 61.334) (end 133.214 60.324992) (width 0.2) (layer "F.Cu") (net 24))
 (segment (start 136.246894 65.24) (end 136.246894 65.76) (width 0.2) (layer "F.Cu") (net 26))
 (segment (start 131.25 62.497) (end 131.25 61.67) (width 0.2) (layer "F.Cu") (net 26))
 (segment (start 132.529702 64.116113) (end 132.699408 63.946407) (width 0.2) (layer "F.Cu") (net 26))
 (segment (start 132.105434 63.691845) (end 131.737738 64.059541) (width 0.2) (layer "F.Cu") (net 26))
 (segment (start 134.806894 66) (end 134.686894 66) (width 0.2) (layer "F.Cu") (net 26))
 (segment (start 132.275141 63.522142) (end 132.275141 63.522141) (width 0.2) (layer "F.Cu") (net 26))
 (segment (start 135.646894 65.24) (end 135.646894 65) (width 0.2) (layer "F.Cu") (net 26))
 (segment (start 132.275141 63.522141) (end 132.105434 63.691845) (width 0.2) (layer "F.Cu") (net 26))
 (segment (start 132.699408 63.946407) (end 132.699407 63.946407) (width 0.2) (layer "F.Cu") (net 26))
 (segment (start 131.398328 64.059542) (end 131.313475 63.974689) (width 0.2) (layer "F.Cu") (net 26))
 (segment (start 135.046894 65.24) (end 135.046894 65.76) (width 0.2) (layer "F.Cu") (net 26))
 (segment (start 132.699407 63.946407) (end 133.236808 63.409005) (width 0.2) (layer "F.Cu") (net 26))
 (segment (start 131.68117 62.92817) (end 131.596318 62.843318) (width 0.2) (layer "F.Cu") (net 26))
 (segment (start 131.313475 63.635277) (end 131.681169 63.26758) (width 0.2) (layer "F.Cu") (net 26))
 (segment (start 135.646894 65) (end 135.646894 64.24) (width 0.2) (layer "F.Cu") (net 26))
 (segment (start 135.406894 64) (end 135.286894 64) (width 0.2) (layer "F.Cu") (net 26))
 (segment (start 136.006894 66) (end 135.886894 66) (width 0.2) (layer "F.Cu") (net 26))
 (segment (start 135.046894 65) (end 135.046894 65.24) (width 0.2) (layer "F.Cu") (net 26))
 (segment (start 133.753 65) (end 133.29338 64.54038) (width 0.2) (layer "F.Cu") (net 26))
 (segment (start 132.162008 64.48381) (end 132.529702 64.116113) (width 0.2) (layer "F.Cu") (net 26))
 (segment (start 132.246861 64.908075) (end 132.162008 64.823222) (width 0.2) (layer "F.Cu") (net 26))
 (segment (start 134.446894 65.76) (end 134.446894 65.24) (width 0.2) (layer "F.Cu") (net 26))
 (segment (start 131.328774 62.575774) (end 131.25 62.497) (width 0.2) (layer "F.Cu") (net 26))
 (segment (start 132.812543 62.984741) (end 132.275141 63.522142) (width 0.2) (layer "F.Cu") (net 26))
 (segment (start 133.236808 63.069594) (end 133.151955 62.984741) (width 0.2) (layer "F.Cu") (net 26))
 (segment (start 135.646894 65.76) (end 135.646894 65.24) (width 0.2) (layer "F.Cu") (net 26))
 (segment (start 140 65) (end 136.486894 65) (width 0.2) (layer "F.Cu") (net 26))
 (segment (start 134.206894 65) (end 134.086894 65) (width 0.2) (layer "F.Cu") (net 26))
 (segment (start 134.086894 65) (end 133.753 65) (width 0.2) (layer "F.Cu") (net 26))
 (segment (start 132.953968 64.54038) (end 132.586271 64.908074) (width 0.2) (layer "F.Cu") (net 26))
 (segment (start 135.046894 64.24) (end 135.046894 65) (width 0.2) (layer "F.Cu") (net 26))
 (segment (start 131.596318 62.843318) (end 131.328774 62.575774) (width 0.2) (layer "F.Cu") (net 26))
 (arc (start 136.486894 65) (mid 136.317188 65.070294) (end 136.246894 65.24) (width 0.2) (layer "F.Cu") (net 26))
 (arc (start 132.586271 64.908074) (mid 132.416566 64.97837) (end 132.246861 64.908075) (width 0.2) (layer "F.Cu") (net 26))
 (arc (start 133.236808 63.409005) (mid 133.307103 63.239299) (end 133.236808 63.069594) (width 0.2) (layer "F.Cu") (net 26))
 (arc (start 134.686894 66) (mid 134.517188 65.929706) (end 134.446894 65.76) (width 0.2) (layer "F.Cu") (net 26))
 (arc (start 131.681169 63.26758) (mid 131.751465 63.097875) (end 131.68117 62.92817) (width 0.2) (layer "F.Cu") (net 26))
 (arc (start 135.046894 65.76) (mid 134.9766 65.929706) (end 134.806894 66) (width 0.2) (layer "F.Cu") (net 26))
 (arc (start 134.446894 65.24) (mid 134.3766 65.070294) (end 134.206894 65) (width 0.2) (layer "F.Cu") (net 26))
 (arc (start 136.246894 65.76) (mid 136.1766 65.929706) (end 136.006894 66) (width 0.2) (layer "F.Cu") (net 26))
 (arc (start 133.151955 62.984741) (mid 132.982249 62.914446) (end 132.812543 62.984741) (width 0.2) (layer "F.Cu") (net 26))
 (arc (start 132.162008 64.823222) (mid 132.091712 64.653515) (end 132.162008 64.48381) (width 0.2) (layer "F.Cu") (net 26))
 (arc (start 135.286894 64) (mid 135.117188 64.070294) (end 135.046894 64.24) (width 0.2) (layer "F.Cu") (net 26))
 (arc (start 135.646894 64.24) (mid 135.5766 64.070294) (end 135.406894 64) (width 0.2) (layer "F.Cu") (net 26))
 (arc (start 131.313475 63.974689) (mid 131.243179 63.804982) (end 131.313475 63.635277) (width 0.2) (layer "F.Cu") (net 26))
 (arc (start 131.737738 64.059541) (mid 131.568033 64.129837) (end 131.398328 64.059542) (width 0.2) (layer "F.Cu") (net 26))
 (arc (start 135.886894 66) (mid 135.717188 65.929706) (end 135.646894 65.76) (width 0.2) (layer "F.Cu") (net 26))
 (arc (start 133.29338 64.54038) (mid 133.123673 64.470084) (end 132.953968 64.54038) (width 0.2) (layer "F.Cu") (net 26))
 (segment (start 129.25 62.497) (end 137.452 70.699) (width 0.2) (layer "F.Cu") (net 21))
 (segment (start 137.452 70.699) (end 144.699 70.699) (width 0.2) (layer "F.Cu") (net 21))
 (segment (start 144.699 70.699) (end 149 75) (width 0.2) (layer "F.Cu") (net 21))
 (segment (start 129.25 61.67) (end 129.25 62.497) (width 0.2) (layer "F.Cu") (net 21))
 (segment (start 164.391 84.849) (end 164.042 84.5) (width 0.2) (layer "F.Cu") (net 7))
 (segment (start 164.391 89.01676) (end 164.391 84.849) (width 0.2) (layer "F.Cu") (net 7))
 (segment (start 155.88 84.5) (end 151.38 80) (width 0.2) (layer "F.Cu") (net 7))
 (segment (start 162.76324 89.691) (end 163.71676 89.691) (width 0.2) (layer "F.Cu") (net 7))
 (segment (start 142.85 105.5) (end 143.419 104.931) (width 0.2) (layer "F.Cu") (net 7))
 (segment (start 148.47676 104.931) (end 152.17355 101.23421) (width 0.2) (layer "F.Cu") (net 7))
 (segment (start 152.17355 101.23421) (end 152.17355 100.28069) (width 0.2) (layer "F.Cu") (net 7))
 (segment (start 163.71676 89.691) (end 164.391 89.01676) (width 0.2) (layer "F.Cu") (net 7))
 (segment (start 143.419 104.931) (end 148.47676 104.931) (width 0.2) (layer "F.Cu") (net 7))
 (segment (start 164.042 84.5) (end 155.88 84.5) (width 0.2) (layer "F.Cu") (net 7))
 (segment (start 152.17355 100.28069) (end 162.76324 89.691) (width 0.2) (layer "F.Cu") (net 7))
 (segment (start 148.75 80) (end 143.25 85.5) (width 0.2) (layer "B.Cu") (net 7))
 (segment (start 151.38 80) (end 148.75 80) (width 0.2) (layer "B.Cu") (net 7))
 (segment (start 143.25 85.5) (end 126.5 85.5) (width 0.2) (layer "B.Cu") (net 7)))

